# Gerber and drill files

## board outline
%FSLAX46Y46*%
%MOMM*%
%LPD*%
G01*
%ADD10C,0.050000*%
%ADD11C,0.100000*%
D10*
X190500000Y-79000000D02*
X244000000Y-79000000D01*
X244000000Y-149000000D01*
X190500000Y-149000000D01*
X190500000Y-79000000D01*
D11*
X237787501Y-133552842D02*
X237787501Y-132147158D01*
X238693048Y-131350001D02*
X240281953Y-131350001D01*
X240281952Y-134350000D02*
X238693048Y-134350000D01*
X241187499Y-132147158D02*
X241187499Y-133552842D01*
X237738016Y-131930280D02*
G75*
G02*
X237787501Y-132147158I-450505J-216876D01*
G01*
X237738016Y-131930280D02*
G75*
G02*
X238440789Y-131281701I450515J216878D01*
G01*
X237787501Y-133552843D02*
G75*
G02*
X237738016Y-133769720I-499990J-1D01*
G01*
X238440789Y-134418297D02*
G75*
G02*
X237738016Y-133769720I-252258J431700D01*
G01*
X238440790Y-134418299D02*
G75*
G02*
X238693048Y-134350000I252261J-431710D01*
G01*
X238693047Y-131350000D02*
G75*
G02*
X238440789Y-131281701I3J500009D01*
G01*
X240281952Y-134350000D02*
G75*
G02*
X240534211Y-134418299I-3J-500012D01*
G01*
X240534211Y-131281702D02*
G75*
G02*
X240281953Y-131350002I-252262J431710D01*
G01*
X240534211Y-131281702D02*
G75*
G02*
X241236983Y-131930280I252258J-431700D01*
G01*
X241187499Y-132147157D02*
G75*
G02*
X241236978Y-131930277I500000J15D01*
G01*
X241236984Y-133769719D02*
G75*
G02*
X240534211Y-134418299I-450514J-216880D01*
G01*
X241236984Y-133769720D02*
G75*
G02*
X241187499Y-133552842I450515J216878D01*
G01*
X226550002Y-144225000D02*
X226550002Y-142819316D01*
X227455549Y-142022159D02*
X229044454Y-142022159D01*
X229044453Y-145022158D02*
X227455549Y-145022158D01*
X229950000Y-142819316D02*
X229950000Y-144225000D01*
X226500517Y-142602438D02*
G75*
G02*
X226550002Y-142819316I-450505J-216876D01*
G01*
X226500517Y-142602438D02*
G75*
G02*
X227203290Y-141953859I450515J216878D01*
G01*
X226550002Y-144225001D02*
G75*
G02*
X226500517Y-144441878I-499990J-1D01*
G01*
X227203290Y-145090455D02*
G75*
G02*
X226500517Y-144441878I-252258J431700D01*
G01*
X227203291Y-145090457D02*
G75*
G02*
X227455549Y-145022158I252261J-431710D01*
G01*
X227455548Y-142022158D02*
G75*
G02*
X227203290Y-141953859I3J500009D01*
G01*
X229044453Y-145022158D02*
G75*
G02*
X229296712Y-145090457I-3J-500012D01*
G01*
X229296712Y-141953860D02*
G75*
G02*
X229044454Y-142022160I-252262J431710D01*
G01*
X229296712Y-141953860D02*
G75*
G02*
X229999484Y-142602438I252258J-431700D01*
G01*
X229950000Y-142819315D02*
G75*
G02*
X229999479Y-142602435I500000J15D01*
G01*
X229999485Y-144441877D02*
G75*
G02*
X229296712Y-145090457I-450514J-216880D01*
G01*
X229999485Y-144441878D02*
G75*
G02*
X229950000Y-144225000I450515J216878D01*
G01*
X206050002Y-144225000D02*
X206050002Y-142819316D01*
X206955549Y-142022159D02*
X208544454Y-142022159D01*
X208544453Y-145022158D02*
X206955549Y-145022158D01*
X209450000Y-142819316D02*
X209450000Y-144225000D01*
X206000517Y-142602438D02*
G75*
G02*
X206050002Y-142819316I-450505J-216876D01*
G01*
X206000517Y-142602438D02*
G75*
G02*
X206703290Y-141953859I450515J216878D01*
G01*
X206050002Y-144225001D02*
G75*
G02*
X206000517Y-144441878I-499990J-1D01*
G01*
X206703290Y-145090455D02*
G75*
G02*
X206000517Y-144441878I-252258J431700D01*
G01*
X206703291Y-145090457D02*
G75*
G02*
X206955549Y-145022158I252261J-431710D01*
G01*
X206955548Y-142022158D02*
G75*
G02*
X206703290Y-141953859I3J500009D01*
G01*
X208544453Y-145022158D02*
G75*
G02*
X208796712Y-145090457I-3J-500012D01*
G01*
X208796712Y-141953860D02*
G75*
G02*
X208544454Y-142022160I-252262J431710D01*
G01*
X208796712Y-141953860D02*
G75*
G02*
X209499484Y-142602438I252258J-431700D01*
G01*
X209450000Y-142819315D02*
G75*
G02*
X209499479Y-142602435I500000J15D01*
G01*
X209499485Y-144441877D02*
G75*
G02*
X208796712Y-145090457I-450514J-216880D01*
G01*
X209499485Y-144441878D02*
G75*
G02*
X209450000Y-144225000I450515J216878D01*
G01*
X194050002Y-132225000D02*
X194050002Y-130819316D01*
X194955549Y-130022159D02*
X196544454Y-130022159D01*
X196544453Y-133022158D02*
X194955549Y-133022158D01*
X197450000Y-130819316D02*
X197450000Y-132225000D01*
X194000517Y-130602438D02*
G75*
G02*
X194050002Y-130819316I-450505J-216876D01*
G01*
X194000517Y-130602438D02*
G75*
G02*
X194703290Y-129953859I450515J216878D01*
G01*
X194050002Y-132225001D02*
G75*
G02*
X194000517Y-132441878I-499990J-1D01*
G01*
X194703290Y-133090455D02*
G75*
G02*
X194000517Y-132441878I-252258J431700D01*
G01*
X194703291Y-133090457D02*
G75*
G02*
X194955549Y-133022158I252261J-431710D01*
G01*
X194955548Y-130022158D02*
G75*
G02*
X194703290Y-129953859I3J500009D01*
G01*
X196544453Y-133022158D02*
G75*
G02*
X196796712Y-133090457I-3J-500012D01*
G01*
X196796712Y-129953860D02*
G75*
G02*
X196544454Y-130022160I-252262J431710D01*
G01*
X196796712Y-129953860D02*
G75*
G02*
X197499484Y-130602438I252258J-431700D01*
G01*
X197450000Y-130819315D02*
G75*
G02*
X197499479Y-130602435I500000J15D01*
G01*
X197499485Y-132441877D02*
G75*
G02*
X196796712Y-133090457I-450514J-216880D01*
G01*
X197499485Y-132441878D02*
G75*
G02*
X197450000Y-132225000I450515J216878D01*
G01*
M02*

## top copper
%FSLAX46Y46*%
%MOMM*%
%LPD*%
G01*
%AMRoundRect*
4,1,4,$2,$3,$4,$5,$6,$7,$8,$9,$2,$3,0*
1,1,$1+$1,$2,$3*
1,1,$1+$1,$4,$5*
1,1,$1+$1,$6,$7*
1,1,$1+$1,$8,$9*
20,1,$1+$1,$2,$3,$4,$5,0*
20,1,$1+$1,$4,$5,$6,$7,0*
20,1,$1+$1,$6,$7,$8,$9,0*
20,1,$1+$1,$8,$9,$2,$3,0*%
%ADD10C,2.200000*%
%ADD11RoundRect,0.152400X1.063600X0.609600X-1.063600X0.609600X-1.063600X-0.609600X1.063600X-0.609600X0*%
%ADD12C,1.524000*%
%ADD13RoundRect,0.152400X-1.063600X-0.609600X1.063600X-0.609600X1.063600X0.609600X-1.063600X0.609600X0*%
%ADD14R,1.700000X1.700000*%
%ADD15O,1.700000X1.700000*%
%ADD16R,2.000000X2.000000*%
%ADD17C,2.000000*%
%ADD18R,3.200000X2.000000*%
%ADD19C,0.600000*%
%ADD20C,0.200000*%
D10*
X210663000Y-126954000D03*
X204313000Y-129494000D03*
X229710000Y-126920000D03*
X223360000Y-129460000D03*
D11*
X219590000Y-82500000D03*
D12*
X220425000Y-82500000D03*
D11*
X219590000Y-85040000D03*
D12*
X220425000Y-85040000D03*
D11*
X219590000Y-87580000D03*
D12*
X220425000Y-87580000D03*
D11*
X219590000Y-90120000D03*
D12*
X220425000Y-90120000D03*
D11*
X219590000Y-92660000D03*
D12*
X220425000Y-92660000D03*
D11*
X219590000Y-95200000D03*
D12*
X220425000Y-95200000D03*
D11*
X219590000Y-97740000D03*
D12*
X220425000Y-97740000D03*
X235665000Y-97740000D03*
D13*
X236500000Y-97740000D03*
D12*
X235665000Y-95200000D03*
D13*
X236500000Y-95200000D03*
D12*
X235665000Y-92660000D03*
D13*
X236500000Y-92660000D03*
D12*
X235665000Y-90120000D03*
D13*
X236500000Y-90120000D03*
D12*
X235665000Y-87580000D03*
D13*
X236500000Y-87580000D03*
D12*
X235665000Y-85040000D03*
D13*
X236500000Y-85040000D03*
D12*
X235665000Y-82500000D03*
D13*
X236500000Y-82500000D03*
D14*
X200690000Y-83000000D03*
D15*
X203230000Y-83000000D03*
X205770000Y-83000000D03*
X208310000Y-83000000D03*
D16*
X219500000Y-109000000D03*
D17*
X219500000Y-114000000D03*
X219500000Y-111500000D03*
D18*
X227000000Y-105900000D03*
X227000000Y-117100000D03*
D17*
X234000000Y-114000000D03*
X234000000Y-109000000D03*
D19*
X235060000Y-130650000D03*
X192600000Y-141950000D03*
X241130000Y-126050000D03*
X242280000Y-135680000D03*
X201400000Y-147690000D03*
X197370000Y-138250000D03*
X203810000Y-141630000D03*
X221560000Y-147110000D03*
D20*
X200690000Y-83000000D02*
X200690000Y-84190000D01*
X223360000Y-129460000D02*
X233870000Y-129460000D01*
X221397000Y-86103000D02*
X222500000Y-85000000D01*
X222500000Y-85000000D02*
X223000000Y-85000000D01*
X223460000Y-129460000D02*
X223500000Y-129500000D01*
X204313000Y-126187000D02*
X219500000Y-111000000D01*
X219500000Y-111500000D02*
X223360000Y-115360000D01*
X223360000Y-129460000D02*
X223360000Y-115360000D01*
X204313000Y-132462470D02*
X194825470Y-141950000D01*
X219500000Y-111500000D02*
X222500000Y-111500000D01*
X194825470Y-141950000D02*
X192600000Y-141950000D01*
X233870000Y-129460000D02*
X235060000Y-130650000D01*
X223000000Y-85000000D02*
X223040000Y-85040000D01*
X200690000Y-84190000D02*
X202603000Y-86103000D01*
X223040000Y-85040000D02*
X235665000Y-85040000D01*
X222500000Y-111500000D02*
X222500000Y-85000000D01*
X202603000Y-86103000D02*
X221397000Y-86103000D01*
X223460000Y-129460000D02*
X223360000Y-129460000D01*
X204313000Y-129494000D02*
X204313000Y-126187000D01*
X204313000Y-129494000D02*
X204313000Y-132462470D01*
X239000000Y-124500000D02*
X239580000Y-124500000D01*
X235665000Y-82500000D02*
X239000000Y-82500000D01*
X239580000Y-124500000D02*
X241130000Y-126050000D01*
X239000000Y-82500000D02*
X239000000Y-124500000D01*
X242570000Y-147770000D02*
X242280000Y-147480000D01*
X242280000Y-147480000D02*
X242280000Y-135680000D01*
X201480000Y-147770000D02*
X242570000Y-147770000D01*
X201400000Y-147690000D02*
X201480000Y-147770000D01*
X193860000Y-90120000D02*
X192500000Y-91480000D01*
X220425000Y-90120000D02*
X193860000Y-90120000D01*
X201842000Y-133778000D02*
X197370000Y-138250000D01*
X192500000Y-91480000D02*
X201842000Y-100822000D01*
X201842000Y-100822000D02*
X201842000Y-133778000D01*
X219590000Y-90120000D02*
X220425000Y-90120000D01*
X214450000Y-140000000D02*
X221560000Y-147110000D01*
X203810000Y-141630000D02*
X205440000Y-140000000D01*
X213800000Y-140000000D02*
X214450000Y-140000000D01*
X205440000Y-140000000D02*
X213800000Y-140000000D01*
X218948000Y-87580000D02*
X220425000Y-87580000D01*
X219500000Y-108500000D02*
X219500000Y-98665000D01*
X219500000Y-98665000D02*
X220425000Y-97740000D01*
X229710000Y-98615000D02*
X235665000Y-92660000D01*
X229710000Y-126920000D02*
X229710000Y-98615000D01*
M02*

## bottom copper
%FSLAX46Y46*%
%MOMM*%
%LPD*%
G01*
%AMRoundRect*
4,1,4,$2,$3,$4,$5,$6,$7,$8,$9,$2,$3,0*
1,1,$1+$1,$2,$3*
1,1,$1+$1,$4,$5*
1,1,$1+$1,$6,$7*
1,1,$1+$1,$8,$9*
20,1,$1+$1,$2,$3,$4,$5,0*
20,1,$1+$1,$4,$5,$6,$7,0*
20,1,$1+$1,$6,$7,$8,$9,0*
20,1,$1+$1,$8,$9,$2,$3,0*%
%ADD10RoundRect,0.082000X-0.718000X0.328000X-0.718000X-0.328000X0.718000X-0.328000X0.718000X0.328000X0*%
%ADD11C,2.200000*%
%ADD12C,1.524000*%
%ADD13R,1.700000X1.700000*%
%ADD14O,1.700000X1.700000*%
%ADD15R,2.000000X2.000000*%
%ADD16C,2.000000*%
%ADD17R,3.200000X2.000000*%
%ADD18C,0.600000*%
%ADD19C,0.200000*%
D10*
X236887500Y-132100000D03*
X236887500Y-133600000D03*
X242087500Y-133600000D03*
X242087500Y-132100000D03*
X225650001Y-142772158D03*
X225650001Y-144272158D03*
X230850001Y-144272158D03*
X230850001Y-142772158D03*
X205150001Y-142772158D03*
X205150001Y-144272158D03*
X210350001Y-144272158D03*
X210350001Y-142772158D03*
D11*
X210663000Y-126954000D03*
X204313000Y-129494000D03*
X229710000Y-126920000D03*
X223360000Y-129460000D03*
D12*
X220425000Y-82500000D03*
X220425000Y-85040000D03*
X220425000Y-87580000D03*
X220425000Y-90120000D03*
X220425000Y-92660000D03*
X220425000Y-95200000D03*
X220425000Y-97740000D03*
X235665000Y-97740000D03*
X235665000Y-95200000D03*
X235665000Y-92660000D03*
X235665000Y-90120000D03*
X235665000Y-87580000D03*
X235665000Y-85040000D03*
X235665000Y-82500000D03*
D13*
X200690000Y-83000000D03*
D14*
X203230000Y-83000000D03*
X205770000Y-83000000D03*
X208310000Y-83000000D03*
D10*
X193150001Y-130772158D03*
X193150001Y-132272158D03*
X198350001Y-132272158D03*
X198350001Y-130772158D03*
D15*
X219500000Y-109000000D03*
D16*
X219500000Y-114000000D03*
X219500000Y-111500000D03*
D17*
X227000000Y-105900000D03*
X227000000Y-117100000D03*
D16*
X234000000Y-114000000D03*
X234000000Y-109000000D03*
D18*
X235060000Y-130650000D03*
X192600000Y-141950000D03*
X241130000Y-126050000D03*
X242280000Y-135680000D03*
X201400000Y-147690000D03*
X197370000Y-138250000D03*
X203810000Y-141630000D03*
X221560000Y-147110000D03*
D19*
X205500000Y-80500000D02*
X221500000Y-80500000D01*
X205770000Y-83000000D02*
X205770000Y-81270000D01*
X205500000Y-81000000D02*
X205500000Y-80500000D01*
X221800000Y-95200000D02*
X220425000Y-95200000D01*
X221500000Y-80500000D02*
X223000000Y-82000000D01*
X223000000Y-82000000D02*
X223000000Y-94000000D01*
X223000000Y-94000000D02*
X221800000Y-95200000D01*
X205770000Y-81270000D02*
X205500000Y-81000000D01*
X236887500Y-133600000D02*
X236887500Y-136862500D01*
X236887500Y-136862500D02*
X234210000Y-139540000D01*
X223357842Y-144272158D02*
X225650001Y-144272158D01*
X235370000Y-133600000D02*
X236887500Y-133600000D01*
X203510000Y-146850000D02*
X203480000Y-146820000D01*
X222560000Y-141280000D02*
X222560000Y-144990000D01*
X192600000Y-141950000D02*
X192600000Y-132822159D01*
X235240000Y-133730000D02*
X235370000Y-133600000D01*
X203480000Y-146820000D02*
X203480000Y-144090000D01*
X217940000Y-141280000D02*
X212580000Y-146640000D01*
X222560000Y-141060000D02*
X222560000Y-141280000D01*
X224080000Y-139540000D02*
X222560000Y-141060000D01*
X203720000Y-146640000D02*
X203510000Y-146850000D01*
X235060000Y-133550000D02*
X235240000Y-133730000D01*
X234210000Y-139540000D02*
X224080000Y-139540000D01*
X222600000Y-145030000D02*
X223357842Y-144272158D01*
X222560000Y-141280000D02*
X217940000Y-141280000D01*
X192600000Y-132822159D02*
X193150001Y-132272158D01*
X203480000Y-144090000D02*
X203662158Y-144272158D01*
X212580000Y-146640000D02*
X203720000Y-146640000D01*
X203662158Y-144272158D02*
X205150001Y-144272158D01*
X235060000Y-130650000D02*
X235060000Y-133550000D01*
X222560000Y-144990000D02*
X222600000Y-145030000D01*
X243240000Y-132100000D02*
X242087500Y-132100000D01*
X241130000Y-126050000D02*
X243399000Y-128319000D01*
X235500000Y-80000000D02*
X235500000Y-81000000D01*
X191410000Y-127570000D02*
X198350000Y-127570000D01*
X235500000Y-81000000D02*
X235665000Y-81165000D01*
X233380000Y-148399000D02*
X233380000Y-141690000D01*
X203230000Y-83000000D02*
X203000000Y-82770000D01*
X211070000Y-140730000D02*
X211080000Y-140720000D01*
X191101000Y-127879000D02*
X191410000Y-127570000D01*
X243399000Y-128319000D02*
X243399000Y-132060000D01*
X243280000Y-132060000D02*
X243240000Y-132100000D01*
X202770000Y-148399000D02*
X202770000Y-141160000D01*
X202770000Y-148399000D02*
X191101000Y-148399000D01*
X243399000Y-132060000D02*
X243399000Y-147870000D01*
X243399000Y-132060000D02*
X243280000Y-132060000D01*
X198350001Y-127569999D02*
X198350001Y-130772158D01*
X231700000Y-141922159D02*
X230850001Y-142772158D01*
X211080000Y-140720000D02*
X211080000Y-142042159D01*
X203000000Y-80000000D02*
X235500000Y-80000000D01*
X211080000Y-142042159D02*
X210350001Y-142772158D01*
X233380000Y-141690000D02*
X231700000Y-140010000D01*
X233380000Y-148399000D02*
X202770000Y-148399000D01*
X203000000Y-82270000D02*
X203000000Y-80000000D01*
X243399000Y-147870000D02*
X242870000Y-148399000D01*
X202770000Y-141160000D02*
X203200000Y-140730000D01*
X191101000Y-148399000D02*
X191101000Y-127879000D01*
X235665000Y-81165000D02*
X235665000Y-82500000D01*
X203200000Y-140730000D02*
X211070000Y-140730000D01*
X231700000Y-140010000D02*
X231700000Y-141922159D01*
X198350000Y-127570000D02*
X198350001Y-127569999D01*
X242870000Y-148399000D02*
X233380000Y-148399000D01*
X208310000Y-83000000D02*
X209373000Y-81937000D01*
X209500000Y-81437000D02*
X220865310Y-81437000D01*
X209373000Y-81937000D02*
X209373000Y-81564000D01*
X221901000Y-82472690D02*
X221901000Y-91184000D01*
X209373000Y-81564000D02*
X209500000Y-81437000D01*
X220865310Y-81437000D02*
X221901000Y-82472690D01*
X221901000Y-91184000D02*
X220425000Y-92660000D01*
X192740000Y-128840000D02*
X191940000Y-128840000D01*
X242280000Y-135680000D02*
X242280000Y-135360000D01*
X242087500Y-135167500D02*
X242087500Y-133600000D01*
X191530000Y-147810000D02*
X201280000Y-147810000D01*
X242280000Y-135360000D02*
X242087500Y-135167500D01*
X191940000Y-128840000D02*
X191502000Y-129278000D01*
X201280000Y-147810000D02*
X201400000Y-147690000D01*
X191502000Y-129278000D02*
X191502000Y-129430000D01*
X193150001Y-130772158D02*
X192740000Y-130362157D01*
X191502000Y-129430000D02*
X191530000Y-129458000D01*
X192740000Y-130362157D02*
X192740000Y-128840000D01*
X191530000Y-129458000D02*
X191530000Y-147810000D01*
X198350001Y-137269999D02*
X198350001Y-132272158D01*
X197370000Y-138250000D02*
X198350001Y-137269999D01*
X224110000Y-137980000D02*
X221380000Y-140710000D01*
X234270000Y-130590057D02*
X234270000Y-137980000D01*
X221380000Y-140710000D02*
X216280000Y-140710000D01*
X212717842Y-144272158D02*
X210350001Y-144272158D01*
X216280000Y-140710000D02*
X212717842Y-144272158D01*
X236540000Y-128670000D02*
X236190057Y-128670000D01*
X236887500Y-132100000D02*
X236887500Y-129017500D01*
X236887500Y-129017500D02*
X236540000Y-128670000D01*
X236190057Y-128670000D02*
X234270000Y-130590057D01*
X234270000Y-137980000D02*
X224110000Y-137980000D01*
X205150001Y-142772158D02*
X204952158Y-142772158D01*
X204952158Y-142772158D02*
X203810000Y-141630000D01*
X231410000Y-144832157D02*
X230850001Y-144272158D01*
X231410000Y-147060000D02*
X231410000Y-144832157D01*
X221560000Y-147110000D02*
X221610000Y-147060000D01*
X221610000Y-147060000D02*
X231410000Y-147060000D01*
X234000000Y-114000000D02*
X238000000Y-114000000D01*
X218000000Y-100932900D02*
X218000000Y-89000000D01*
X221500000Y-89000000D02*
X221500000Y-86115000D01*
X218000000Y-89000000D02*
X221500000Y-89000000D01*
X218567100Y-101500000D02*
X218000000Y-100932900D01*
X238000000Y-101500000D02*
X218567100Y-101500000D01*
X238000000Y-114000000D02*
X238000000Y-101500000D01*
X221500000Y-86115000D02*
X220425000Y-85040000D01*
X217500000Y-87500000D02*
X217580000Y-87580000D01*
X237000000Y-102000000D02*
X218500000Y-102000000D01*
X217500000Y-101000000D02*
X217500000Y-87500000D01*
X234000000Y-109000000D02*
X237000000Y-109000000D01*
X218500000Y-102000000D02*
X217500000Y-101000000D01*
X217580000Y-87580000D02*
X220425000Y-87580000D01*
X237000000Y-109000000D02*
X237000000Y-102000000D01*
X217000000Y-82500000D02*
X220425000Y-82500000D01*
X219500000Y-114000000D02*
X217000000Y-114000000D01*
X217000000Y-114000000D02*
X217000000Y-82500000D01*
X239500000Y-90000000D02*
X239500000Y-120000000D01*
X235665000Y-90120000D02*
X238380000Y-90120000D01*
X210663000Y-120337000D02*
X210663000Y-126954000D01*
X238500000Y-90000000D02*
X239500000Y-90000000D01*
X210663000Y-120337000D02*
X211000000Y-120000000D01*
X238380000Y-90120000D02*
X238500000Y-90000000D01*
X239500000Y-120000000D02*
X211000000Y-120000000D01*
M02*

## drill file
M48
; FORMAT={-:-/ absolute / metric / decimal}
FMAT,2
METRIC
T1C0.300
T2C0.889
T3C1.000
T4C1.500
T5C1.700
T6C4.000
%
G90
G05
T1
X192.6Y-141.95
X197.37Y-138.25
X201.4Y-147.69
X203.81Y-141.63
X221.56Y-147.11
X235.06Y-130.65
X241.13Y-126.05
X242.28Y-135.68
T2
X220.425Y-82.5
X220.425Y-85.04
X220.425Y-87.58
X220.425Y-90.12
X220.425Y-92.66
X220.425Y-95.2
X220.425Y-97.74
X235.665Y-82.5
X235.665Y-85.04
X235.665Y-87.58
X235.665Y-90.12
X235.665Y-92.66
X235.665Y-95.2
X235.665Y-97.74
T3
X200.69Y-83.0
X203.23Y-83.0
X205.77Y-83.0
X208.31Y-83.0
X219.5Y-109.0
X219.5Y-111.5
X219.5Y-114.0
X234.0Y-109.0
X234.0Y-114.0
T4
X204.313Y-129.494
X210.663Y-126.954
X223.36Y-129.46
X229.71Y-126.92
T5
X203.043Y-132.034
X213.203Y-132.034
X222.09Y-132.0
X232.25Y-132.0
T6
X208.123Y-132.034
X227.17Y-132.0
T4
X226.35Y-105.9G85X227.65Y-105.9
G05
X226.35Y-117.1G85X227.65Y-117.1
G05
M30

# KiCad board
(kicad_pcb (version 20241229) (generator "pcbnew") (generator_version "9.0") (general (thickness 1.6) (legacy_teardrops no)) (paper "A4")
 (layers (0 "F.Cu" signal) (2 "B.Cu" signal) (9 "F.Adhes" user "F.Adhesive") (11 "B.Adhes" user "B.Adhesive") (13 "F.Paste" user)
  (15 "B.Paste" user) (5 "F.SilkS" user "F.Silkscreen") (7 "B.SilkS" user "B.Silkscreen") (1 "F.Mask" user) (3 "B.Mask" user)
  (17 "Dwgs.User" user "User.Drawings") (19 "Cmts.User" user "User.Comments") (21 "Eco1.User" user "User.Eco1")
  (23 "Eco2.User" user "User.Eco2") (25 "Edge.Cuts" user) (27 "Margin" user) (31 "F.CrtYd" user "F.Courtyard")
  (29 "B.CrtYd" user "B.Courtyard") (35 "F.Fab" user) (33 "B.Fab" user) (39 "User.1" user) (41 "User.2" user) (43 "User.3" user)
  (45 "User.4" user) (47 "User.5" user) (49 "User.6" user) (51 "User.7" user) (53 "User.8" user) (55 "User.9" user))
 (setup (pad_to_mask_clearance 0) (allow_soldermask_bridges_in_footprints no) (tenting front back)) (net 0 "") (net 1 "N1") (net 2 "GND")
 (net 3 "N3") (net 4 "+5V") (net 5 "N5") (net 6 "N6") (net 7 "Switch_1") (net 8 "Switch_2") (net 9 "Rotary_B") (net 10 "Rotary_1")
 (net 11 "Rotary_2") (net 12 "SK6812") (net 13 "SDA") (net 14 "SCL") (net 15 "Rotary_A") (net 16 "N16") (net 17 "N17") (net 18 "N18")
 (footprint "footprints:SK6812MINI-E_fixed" (layer "F.Cu") (at 239.487499 132.952842)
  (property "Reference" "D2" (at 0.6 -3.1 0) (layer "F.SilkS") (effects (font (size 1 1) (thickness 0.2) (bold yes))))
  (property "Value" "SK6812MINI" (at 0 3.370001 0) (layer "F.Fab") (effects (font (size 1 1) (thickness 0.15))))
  (fp_line (start -1.699998 0.6) (end -1.699998 -0.805684) (stroke (width 0.1) (type solid)) (layer "Edge.Cuts"))
  (fp_line (start -0.794451 -1.602841) (end 0.794454 -1.602841) (stroke (width 0.1) (type solid)) (layer "Edge.Cuts"))
  (fp_line (start 0.794453 1.397158) (end -0.794451 1.397158) (stroke (width 0.1) (type solid)) (layer "Edge.Cuts"))
  (fp_line (start 1.7 -0.805684) (end 1.7 0.6) (stroke (width 0.1) (type solid)) (layer "Edge.Cuts"))
  (fp_arc (start -1.749483 -1.022562) (mid -1.712526 -0.91691) (end -1.699998 -0.805684) (stroke (width 0.1) (type solid))
   (layer "Edge.Cuts"))
  (fp_arc (start -1.749483 -1.022562) (mid -1.63807 -1.606877) (end -1.04671 -1.671141) (stroke (width 0.1) (type solid))
   (layer "Edge.Cuts"))
  (fp_arc (start -1.699998 0.600001) (mid -1.712526 0.711226) (end -1.749483 0.816878) (stroke (width 0.1) (type solid)) (layer "Edge.Cuts"))
  (fp_arc (start -1.04671 1.465455) (mid -1.638069 1.401192) (end -1.749483 0.816878) (stroke (width 0.1) (type solid)) (layer "Edge.Cuts"))
  (fp_arc (start -1.046709 1.465457) (mid -0.925121 1.414535) (end -0.794451 1.397158) (stroke (width 0.1) (type solid)) (layer "Edge.Cuts"))
  (fp_arc (start -0.794452 -1.602842) (mid -0.925122 -1.620219) (end -1.04671 -1.671141) (stroke (width 0.1) (type solid))
   (layer "Edge.Cuts"))
  (fp_arc (start 0.794453 1.397158) (mid 0.925124 1.414535) (end 1.046712 1.465457) (stroke (width 0.1) (type solid)) (layer "Edge.Cuts"))
  (fp_arc (start 1.046712 -1.67114) (mid 0.925124 -1.620218) (end 0.794454 -1.602841) (stroke (width 0.1) (type solid)) (layer "Edge.Cuts"))
  (fp_arc (start 1.046712 -1.67114) (mid 1.638072 -1.606876) (end 1.749485 -1.022562) (stroke (width 0.1) (type solid)) (layer "Edge.Cuts"))
  (fp_arc (start 1.7 -0.805685) (mid 1.712528 -0.91691) (end 1.749485 -1.022562) (stroke (width 0.1) (type solid)) (layer "Edge.Cuts"))
  (fp_arc (start 1.749485 0.816877) (mid 1.638073 1.401193) (end 1.046712 1.465457) (stroke (width 0.1) (type solid)) (layer "Edge.Cuts"))
  (fp_arc (start 1.749485 0.816878) (mid 1.712528 0.711226) (end 1.7 0.6) (stroke (width 0.1) (type solid)) (layer "Edge.Cuts"))
  (pad "1" smd roundrect (at -2.599999 -0.852842 270) (size 0.82 1.6) (layers "B.Cu" "B.Mask" "B.Paste") (roundrect_rratio 0.1) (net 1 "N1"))
  (pad "2" smd roundrect (at -2.599999 0.647158 270) (size 0.82 1.6) (layers "B.Cu" "B.Mask" "B.Paste") (roundrect_rratio 0.1) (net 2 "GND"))
  (pad "3" smd roundrect (at 2.600001 0.647158 270) (size 0.82 1.6) (layers "B.Cu" "B.Mask" "B.Paste") (roundrect_rratio 0.1) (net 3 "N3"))
  (pad "4" smd roundrect (at 2.600001 -0.852842 270) (size 0.82 1.6) (layers "B.Cu" "B.Mask" "B.Paste") (roundrect_rratio 0.1) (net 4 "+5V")))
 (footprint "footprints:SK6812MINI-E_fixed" (layer "F.Cu") (at 228.25 143.625)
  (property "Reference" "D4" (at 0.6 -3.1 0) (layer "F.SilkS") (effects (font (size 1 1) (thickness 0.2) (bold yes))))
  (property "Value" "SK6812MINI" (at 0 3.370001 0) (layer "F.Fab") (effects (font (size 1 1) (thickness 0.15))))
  (fp_line (start -1.699998 0.6) (end -1.699998 -0.805684) (stroke (width 0.1) (type solid)) (layer "Edge.Cuts"))
  (fp_line (start -0.794451 -1.602841) (end 0.794454 -1.602841) (stroke (width 0.1) (type solid)) (layer "Edge.Cuts"))
  (fp_line (start 0.794453 1.397158) (end -0.794451 1.397158) (stroke (width 0.1) (type solid)) (layer "Edge.Cuts"))
  (fp_line (start 1.7 -0.805684) (end 1.7 0.6) (stroke (width 0.1) (type solid)) (layer "Edge.Cuts"))
  (fp_arc (start -1.749483 -1.022562) (mid -1.712526 -0.91691) (end -1.699998 -0.805684) (stroke (width 0.1) (type solid))
   (layer "Edge.Cuts"))
  (fp_arc (start -1.749483 -1.022562) (mid -1.63807 -1.606877) (end -1.04671 -1.671141) (stroke (width 0.1) (type solid))
   (layer "Edge.Cuts"))
  (fp_arc (start -1.699998 0.600001) (mid -1.712526 0.711226) (end -1.749483 0.816878) (stroke (width 0.1) (type solid)) (layer "Edge.Cuts"))
  (fp_arc (start -1.04671 1.465455) (mid -1.638069 1.401192) (end -1.749483 0.816878) (stroke (width 0.1) (type solid)) (layer "Edge.Cuts"))
  (fp_arc (start -1.046709 1.465457) (mid -0.925121 1.414535) (end -0.794451 1.397158) (stroke (width 0.1) (type solid)) (layer "Edge.Cuts"))
  (fp_arc (start -0.794452 -1.602842) (mid -0.925122 -1.620219) (end -1.04671 -1.671141) (stroke (width 0.1) (type solid))
   (layer "Edge.Cuts"))
  (fp_arc (start 0.794453 1.397158) (mid 0.925124 1.414535) (end 1.046712 1.465457) (stroke (width 0.1) (type solid)) (layer "Edge.Cuts"))
  (fp_arc (start 1.046712 -1.67114) (mid 0.925124 -1.620218) (end 0.794454 -1.602841) (stroke (width 0.1) (type solid)) (layer "Edge.Cuts"))
  (fp_arc (start 1.046712 -1.67114) (mid 1.638072 -1.606876) (end 1.749485 -1.022562) (stroke (width 0.1) (type solid)) (layer "Edge.Cuts"))
  (fp_arc (start 1.7 -0.805685) (mid 1.712528 -0.91691) (end 1.749485 -1.022562) (stroke (width 0.1) (type solid)) (layer "Edge.Cuts"))
  (fp_arc (start 1.749485 0.816877) (mid 1.638073 1.401193) (end 1.046712 1.465457) (stroke (width 0.1) (type solid)) (layer "Edge.Cuts"))
  (fp_arc (start 1.749485 0.816878) (mid 1.712528 0.711226) (end 1.7 0.6) (stroke (width 0.1) (type solid)) (layer "Edge.Cuts"))
  (pad "1" smd roundrect (at -2.599999 -0.852842 270) (size 0.82 1.6) (layers "B.Cu" "B.Mask" "B.Paste") (roundrect_rratio 0.1) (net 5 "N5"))
  (pad "2" smd roundrect (at -2.599999 0.647158 270) (size 0.82 1.6) (layers "B.Cu" "B.Mask" "B.Paste") (roundrect_rratio 0.1) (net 2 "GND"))
  (pad "3" smd roundrect (at 2.600001 0.647158 270) (size 0.82 1.6) (layers "B.Cu" "B.Mask" "B.Paste") (roundrect_rratio 0.1) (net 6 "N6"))
  (pad "4" smd roundrect (at 2.600001 -0.852842 270) (size 0.82 1.6) (layers "B.Cu" "B.Mask" "B.Paste") (roundrect_rratio 0.1) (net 4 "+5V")))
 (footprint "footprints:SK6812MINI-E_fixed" (layer "F.Cu") (at 207.75 143.625)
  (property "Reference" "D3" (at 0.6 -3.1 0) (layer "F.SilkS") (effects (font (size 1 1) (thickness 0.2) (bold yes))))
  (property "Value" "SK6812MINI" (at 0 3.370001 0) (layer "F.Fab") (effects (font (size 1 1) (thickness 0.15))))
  (fp_line (start -1.699998 0.6) (end -1.699998 -0.805684) (stroke (width 0.1) (type solid)) (layer "Edge.Cuts"))
  (fp_line (start -0.794451 -1.602841) (end 0.794454 -1.602841) (stroke (width 0.1) (type solid)) (layer "Edge.Cuts"))
  (fp_line (start 0.794453 1.397158) (end -0.794451 1.397158) (stroke (width 0.1) (type solid)) (layer "Edge.Cuts"))
  (fp_line (start 1.7 -0.805684) (end 1.7 0.6) (stroke (width 0.1) (type solid)) (layer "Edge.Cuts"))
  (fp_arc (start -1.749483 -1.022562) (mid -1.712526 -0.91691) (end -1.699998 -0.805684) (stroke (width 0.1) (type solid))
   (layer "Edge.Cuts"))
  (fp_arc (start -1.749483 -1.022562) (mid -1.63807 -1.606877) (end -1.04671 -1.671141) (stroke (width 0.1) (type solid))
   (layer "Edge.Cuts"))
  (fp_arc (start -1.699998 0.600001) (mid -1.712526 0.711226) (end -1.749483 0.816878) (stroke (width 0.1) (type solid)) (layer "Edge.Cuts"))
  (fp_arc (start -1.04671 1.465455) (mid -1.638069 1.401192) (end -1.749483 0.816878) (stroke (width 0.1) (type solid)) (layer "Edge.Cuts"))
  (fp_arc (start -1.046709 1.465457) (mid -0.925121 1.414535) (end -0.794451 1.397158) (stroke (width 0.1) (type solid)) (layer "Edge.Cuts"))
  (fp_arc (start -0.794452 -1.602842) (mid -0.925122 -1.620219) (end -1.04671 -1.671141) (stroke (width 0.1) (type solid))
   (layer "Edge.Cuts"))
  (fp_arc (start 0.794453 1.397158) (mid 0.925124 1.414535) (end 1.046712 1.465457) (stroke (width 0.1) (type solid)) (layer "Edge.Cuts"))
  (fp_arc (start 1.046712 -1.67114) (mid 0.925124 -1.620218) (end 0.794454 -1.602841) (stroke (width 0.1) (type solid)) (layer "Edge.Cuts"))
  (fp_arc (start 1.046712 -1.67114) (mid 1.638072 -1.606876) (end 1.749485 -1.022562) (stroke (width 0.1) (type solid)) (layer "Edge.Cuts"))
  (fp_arc (start 1.7 -0.805685) (mid 1.712528 -0.91691) (end 1.749485 -1.022562) (stroke (width 0.1) (type solid)) (layer "Edge.Cuts"))
  (fp_arc (start 1.749485 0.816877) (mid 1.638073 1.401193) (end 1.046712 1.465457) (stroke (width 0.1) (type solid)) (layer "Edge.Cuts"))
  (fp_arc (start 1.749485 0.816878) (mid 1.712528 0.711226) (end 1.7 0.6) (stroke (width 0.1) (type solid)) (layer "Edge.Cuts"))
  (pad "1" smd roundrect (at -2.599999 -0.852842 270) (size 0.82 1.6) (layers "B.Cu" "B.Mask" "B.Paste") (roundrect_rratio 0.1) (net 6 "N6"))
  (pad "2" smd roundrect (at -2.599999 0.647158 270) (size 0.82 1.6) (layers "B.Cu" "B.Mask" "B.Paste") (roundrect_rratio 0.1) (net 2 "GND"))
  (pad "3" smd roundrect (at 2.600001 0.647158 270) (size 0.82 1.6) (layers "B.Cu" "B.Mask" "B.Paste") (roundrect_rratio 0.1) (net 1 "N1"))
  (pad "4" smd roundrect (at 2.600001 -0.852842 270) (size 0.82 1.6) (layers "B.Cu" "B.Mask" "B.Paste") (roundrect_rratio 0.1) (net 4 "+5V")))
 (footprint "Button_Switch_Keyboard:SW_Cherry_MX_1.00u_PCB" (layer "F.Cu") (at 210.663 126.954)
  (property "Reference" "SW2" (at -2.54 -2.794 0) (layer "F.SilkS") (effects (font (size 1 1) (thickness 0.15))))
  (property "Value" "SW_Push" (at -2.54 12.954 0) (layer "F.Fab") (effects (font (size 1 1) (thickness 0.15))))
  (pad "" np_thru_hole circle (at -7.62 5.08) (size 1.7 1.7) (drill 1.7) (layers "*.Cu" "*.Mask"))
  (pad "" np_thru_hole circle (at -2.54 5.08) (size 4 4) (drill 4) (layers "*.Cu" "*.Mask"))
  (pad "" np_thru_hole circle (at 2.54 5.08) (size 1.7 1.7) (drill 1.7) (layers "*.Cu" "*.Mask"))
  (pad "1" thru_hole circle (at 0 0) (size 2.2 2.2) (drill 1.5) (layers "*.Cu" "*.Mask") (remove_unused_layers no) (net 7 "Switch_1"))
  (pad "2" thru_hole circle (at -6.35 2.54) (size 2.2 2.2) (drill 1.5) (layers "*.Cu" "*.Mask") (remove_unused_layers no) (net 2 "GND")))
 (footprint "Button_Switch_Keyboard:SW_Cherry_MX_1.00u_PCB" (layer "F.Cu") (at 229.71 126.92)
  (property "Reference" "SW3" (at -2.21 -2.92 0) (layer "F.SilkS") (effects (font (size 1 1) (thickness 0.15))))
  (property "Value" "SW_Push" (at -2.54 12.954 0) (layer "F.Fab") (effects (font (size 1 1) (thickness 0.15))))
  (pad "" np_thru_hole circle (at -7.62 5.08) (size 1.7 1.7) (drill 1.7) (layers "*.Cu" "*.Mask"))
  (pad "" np_thru_hole circle (at -2.54 5.08) (size 4 4) (drill 4) (layers "*.Cu" "*.Mask"))
  (pad "" np_thru_hole circle (at 2.54 5.08) (size 1.7 1.7) (drill 1.7) (layers "*.Cu" "*.Mask"))
  (pad "1" thru_hole circle (at 0 0) (size 2.2 2.2) (drill 1.5) (layers "*.Cu" "*.Mask") (remove_unused_layers no) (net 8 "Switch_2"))
  (pad "2" thru_hole circle (at -6.35 2.54) (size 2.2 2.2) (drill 1.5) (layers "*.Cu" "*.Mask") (remove_unused_layers no) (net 2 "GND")))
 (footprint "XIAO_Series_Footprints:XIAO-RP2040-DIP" (layer "F.Cu") (at 228.045 90.12 90)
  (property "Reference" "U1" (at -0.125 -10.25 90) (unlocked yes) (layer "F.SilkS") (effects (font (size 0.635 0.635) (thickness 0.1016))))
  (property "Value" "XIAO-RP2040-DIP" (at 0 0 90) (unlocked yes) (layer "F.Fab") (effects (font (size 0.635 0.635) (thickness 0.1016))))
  (pad "1" smd roundrect (at 7.62 -8.455 180) (size 2.432 1.524) (layers "F.Cu" "F.Mask") (roundrect_rratio 0.1) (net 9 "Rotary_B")
   (thermal_bridge_angle 45))
  (pad "1" thru_hole circle (at 7.62 -7.62 180) (size 1.524 1.524) (drill 0.889) (layers "*.Cu" "*.Mask") (remove_unused_layers no)
   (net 9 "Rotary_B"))
  (pad "2" smd roundrect (at 5.08 -8.455 180) (size 2.432 1.524) (layers "F.Cu" "F.Mask") (roundrect_rratio 0.1) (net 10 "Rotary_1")
   (thermal_bridge_angle 45))
  (pad "2" thru_hole circle (at 5.08 -7.62 180) (size 1.524 1.524) (drill 0.889) (layers "*.Cu" "*.Mask") (remove_unused_layers no)
   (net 10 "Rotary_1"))
  (pad "3" smd roundrect (at 2.54 -8.455 180) (size 2.432 1.524) (layers "F.Cu" "F.Mask") (roundrect_rratio 0.1) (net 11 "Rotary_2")
   (thermal_bridge_angle 45))
  (pad "3" thru_hole circle (at 2.54 -7.62 180) (size 1.524 1.524) (drill 0.889) (layers "*.Cu" "*.Mask") (remove_unused_layers no)
   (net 11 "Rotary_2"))
  (pad "4" smd roundrect (at 0 -8.455 180) (size 2.432 1.524) (layers "F.Cu" "F.Mask") (roundrect_rratio 0.1) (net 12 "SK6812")
   (thermal_bridge_angle 45))
  (pad "4" thru_hole circle (at 0 -7.62 180) (size 1.524 1.524) (drill 0.889) (layers "*.Cu" "*.Mask") (remove_unused_layers no)
   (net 12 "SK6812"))
  (pad "5" smd roundrect (at -2.54 -8.455 180) (size 2.432 1.524) (layers "F.Cu" "F.Mask") (roundrect_rratio 0.1) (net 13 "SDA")
   (thermal_bridge_angle 45))
  (pad "5" thru_hole circle (at -2.54 -7.62 180) (size 1.524 1.524) (drill 0.889) (layers "*.Cu" "*.Mask") (remove_unused_layers no)
   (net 13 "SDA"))
  (pad "6" smd roundrect (at -5.08 -8.455 180) (size 2.432 1.524) (layers "F.Cu" "F.Mask") (roundrect_rratio 0.1) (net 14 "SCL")
   (thermal_bridge_angle 45))
  (pad "6" thru_hole circle (at -5.08 -7.62 180) (size 1.524 1.524) (drill 0.889) (layers "*.Cu" "*.Mask") (remove_unused_layers no)
   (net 14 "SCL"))
  (pad "7" smd roundrect (at -7.62 -8.455 180) (size 2.432 1.524) (layers "F.Cu" "F.Mask") (roundrect_rratio 0.1) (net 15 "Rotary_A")
   (thermal_bridge_angle 45))
  (pad "7" thru_hole circle (at -7.62 -7.62 180) (size 1.524 1.524) (drill 0.889) (layers "*.Cu" "*.Mask") (remove_unused_layers no)
   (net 15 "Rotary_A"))
  (pad "8" thru_hole circle (at -7.62 7.62) (size 1.524 1.524) (drill 0.889) (layers "*.Cu" "*.Mask") (remove_unused_layers no)
   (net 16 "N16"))
  (pad "8" smd roundrect (at -7.62 8.455) (size 2.432 1.524) (layers "F.Cu" "F.Mask") (roundrect_rratio 0.1) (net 16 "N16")
   (thermal_bridge_angle 45))
  (pad "9" thru_hole circle (at -5.08 7.62) (size 1.524 1.524) (drill 0.889) (layers "*.Cu" "*.Mask") (remove_unused_layers no)
   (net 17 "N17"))
  (pad "9" smd roundrect (at -5.08 8.455) (size 2.432 1.524) (layers "F.Cu" "F.Mask") (roundrect_rratio 0.1) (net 17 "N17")
   (thermal_bridge_angle 45))
  (pad "10" thru_hole circle (at -2.54 7.62) (size 1.524 1.524) (drill 0.889) (layers "*.Cu" "*.Mask") (remove_unused_layers no)
   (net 8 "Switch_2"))
  (pad "10" smd roundrect (at -2.54 8.455) (size 2.432 1.524) (layers "F.Cu" "F.Mask") (roundrect_rratio 0.1) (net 8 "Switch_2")
   (thermal_bridge_angle 45))
  (pad "11" thru_hole circle (at 0 7.62) (size 1.524 1.524) (drill 0.889) (layers "*.Cu" "*.Mask") (remove_unused_layers no)
   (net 7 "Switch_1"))
  (pad "11" smd roundrect (at 0 8.455) (size 2.432 1.524) (layers "F.Cu" "F.Mask") (roundrect_rratio 0.1) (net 7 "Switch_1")
   (thermal_bridge_angle 45))
  (pad "12" thru_hole circle (at 2.54 7.62) (size 1.524 1.524) (drill 0.889) (layers "*.Cu" "*.Mask") (remove_unused_layers no)
   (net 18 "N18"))
  (pad "12" smd roundrect (at 2.54 8.455) (size 2.432 1.524) (layers "F.Cu" "F.Mask") (roundrect_rratio 0.1) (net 18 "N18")
   (thermal_bridge_angle 45))
  (pad "13" thru_hole circle (at 5.08 7.62) (size 1.524 1.524) (drill 0.889) (layers "*.Cu" "*.Mask") (remove_unused_layers no)
   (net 2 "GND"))
  (pad "13" smd roundrect (at 5.08 8.455) (size 2.432 1.524) (layers "F.Cu" "F.Mask") (roundrect_rratio 0.1) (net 2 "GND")
   (thermal_bridge_angle 45))
  (pad "14" thru_hole circle (at 7.62 7.62) (size 1.524 1.524) (drill 0.889) (layers "*.Cu" "*.Mask") (remove_unused_layers no)
   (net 4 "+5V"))
  (pad "14" smd roundrect (at 7.62 8.455) (size 2.432 1.524) (layers "F.Cu" "F.Mask") (roundrect_rratio 0.1) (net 4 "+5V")
   (thermal_bridge_angle 45)))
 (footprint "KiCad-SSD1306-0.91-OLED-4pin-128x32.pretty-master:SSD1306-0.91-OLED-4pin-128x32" (layer "F.Cu") (at 198.5 119.5 90)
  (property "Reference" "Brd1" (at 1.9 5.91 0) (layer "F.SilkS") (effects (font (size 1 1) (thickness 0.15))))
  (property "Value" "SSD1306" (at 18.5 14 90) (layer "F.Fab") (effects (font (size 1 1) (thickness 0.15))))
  (pad "1" thru_hole rect (at 36.5 2.19 90) (size 1.7 1.7) (drill 1) (layers "*.Cu" "*.Mask") (remove_unused_layers no) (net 2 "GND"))
  (pad "2" thru_hole oval (at 36.5 4.73 90) (size 1.7 1.7) (drill 1) (layers "*.Cu" "*.Mask") (remove_unused_layers no) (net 4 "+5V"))
  (pad "3" thru_hole oval (at 36.5 7.27 90) (size 1.7 1.7) (drill 1) (layers "*.Cu" "*.Mask") (remove_unused_layers no) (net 14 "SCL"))
  (pad "4" thru_hole oval (at 36.5 9.81 90) (size 1.7 1.7) (drill 1) (layers "*.Cu" "*.Mask") (remove_unused_layers no) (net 13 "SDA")))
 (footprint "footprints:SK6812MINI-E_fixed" (layer "F.Cu") (at 195.75 131.625)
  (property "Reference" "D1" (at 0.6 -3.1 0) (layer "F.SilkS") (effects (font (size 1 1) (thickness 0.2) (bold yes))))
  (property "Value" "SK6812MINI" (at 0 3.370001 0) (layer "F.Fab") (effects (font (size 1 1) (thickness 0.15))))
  (fp_line (start -1.699998 0.6) (end -1.699998 -0.805684) (stroke (width 0.1) (type solid)) (layer "Edge.Cuts"))
  (fp_line (start -0.794451 -1.602841) (end 0.794454 -1.602841) (stroke (width 0.1) (type solid)) (layer "Edge.Cuts"))
  (fp_line (start 0.794453 1.397158) (end -0.794451 1.397158) (stroke (width 0.1) (type solid)) (layer "Edge.Cuts"))
  (fp_line (start 1.7 -0.805684) (end 1.7 0.6) (stroke (width 0.1) (type solid)) (layer "Edge.Cuts"))
  (fp_arc (start -1.749483 -1.022562) (mid -1.712526 -0.91691) (end -1.699998 -0.805684) (stroke (width 0.1) (type solid))
   (layer "Edge.Cuts"))
  (fp_arc (start -1.749483 -1.022562) (mid -1.63807 -1.606877) (end -1.04671 -1.671141) (stroke (width 0.1) (type solid))
   (layer "Edge.Cuts"))
  (fp_arc (start -1.699998 0.600001) (mid -1.712526 0.711226) (end -1.749483 0.816878) (stroke (width 0.1) (type solid)) (layer "Edge.Cuts"))
  (fp_arc (start -1.04671 1.465455) (mid -1.638069 1.401192) (end -1.749483 0.816878) (stroke (width 0.1) (type solid)) (layer "Edge.Cuts"))
  (fp_arc (start -1.046709 1.465457) (mid -0.925121 1.414535) (end -0.794451 1.397158) (stroke (width 0.1) (type solid)) (layer "Edge.Cuts"))
  (fp_arc (start -0.794452 -1.602842) (mid -0.925122 -1.620219) (end -1.04671 -1.671141) (stroke (width 0.1) (type solid))
   (layer "Edge.Cuts"))
  (fp_arc (start 0.794453 1.397158) (mid 0.925124 1.414535) (end 1.046712 1.465457) (stroke (width 0.1) (type solid)) (layer "Edge.Cuts"))
  (fp_arc (start 1.046712 -1.67114) (mid 0.925124 -1.620218) (end 0.794454 -1.602841) (stroke (width 0.1) (type solid)) (layer "Edge.Cuts"))
  (fp_arc (start 1.046712 -1.67114) (mid 1.638072 -1.606876) (end 1.749485 -1.022562) (stroke (width 0.1) (type solid)) (layer "Edge.Cuts"))
  (fp_arc (start 1.7 -0.805685) (mid 1.712528 -0.91691) (end 1.749485 -1.022562) (stroke (width 0.1) (type solid)) (layer "Edge.Cuts"))
  (fp_arc (start 1.749485 0.816877) (mid 1.638073 1.401193) (end 1.046712 1.465457) (stroke (width 0.1) (type solid)) (layer "Edge.Cuts"))
  (fp_arc (start 1.749485 0.816878) (mid 1.712528 0.711226) (end 1.7 0.6) (stroke (width 0.1) (type solid)) (layer "Edge.Cuts"))
  (pad "1" smd roundrect (at -2.599999 -0.852842 270) (size 0.82 1.6) (layers "B.Cu" "B.Mask" "B.Paste") (roundrect_rratio 0.1) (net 3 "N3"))
  (pad "2" smd roundrect (at -2.599999 0.647158 270) (size 0.82 1.6) (layers "B.Cu" "B.Mask" "B.Paste") (roundrect_rratio 0.1) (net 2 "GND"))
  (pad "3" smd roundrect (at 2.600001 0.647158 270) (size 0.82 1.6) (layers "B.Cu" "B.Mask" "B.Paste") (roundrect_rratio 0.1)
   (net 12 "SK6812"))
  (pad "4" smd roundrect (at 2.600001 -0.852842 270) (size 0.82 1.6) (layers "B.Cu" "B.Mask" "B.Paste") (roundrect_rratio 0.1) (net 4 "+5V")))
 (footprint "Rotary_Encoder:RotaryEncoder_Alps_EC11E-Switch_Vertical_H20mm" (layer "F.Cu") (at 219.5 109)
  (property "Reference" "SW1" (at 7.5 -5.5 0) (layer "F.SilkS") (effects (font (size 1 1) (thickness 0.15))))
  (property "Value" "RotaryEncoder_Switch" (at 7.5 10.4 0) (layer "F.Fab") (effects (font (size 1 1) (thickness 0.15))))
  (pad "A" thru_hole rect (at 0 0) (size 2 2) (drill 1) (layers "*.Cu" "*.Mask") (remove_unused_layers no) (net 15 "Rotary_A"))
  (pad "B" thru_hole circle (at 0 5) (size 2 2) (drill 1) (layers "*.Cu" "*.Mask") (remove_unused_layers no) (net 9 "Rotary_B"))
  (pad "C" thru_hole circle (at 0 2.5) (size 2 2) (drill 1) (layers "*.Cu" "*.Mask") (remove_unused_layers no) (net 2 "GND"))
  (pad "MP" thru_hole rect (at 7.5 -3.1) (size 3.2 2) (drill oval 2.8 1.5) (layers "*.Cu" "*.Mask") (remove_unused_layers no))
  (pad "MP" thru_hole rect (at 7.5 8.1) (size 3.2 2) (drill oval 2.8 1.5) (layers "*.Cu" "*.Mask") (remove_unused_layers no))
  (pad "S1" thru_hole circle (at 14.5 5) (size 2 2) (drill 1) (layers "*.Cu" "*.Mask") (remove_unused_layers no) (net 10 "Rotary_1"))
  (pad "S2" thru_hole circle (at 14.5 0) (size 2 2) (drill 1) (layers "*.Cu" "*.Mask") (remove_unused_layers no) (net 11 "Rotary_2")))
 (gr_rect (start 190.5 79) (end 244 149) (stroke (width 0.05) (type default)) (fill no) (layer "Edge.Cuts"))
 (segment (start 205.5 80.5) (end 221.5 80.5) (width 0.2) (layer "B.Cu") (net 14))
 (segment (start 205.77 83) (end 205.77 81.27) (width 0.2) (layer "B.Cu") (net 14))
 (segment (start 205.5 81) (end 205.5 80.5) (width 0.2) (layer "B.Cu") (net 14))
 (segment (start 221.8 95.2) (end 220.425 95.2) (width 0.2) (layer "B.Cu") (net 14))
 (segment (start 221.5 80.5) (end 223 82) (width 0.2) (layer "B.Cu") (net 14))
 (segment (start 223 82) (end 223 94) (width 0.2) (layer "B.Cu") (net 14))
 (segment (start 223 94) (end 221.8 95.2) (width 0.2) (layer "B.Cu") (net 14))
 (segment (start 205.77 81.27) (end 205.5 81) (width 0.2) (layer "B.Cu") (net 14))
 (segment (start 200.69 83) (end 200.69 84.19) (width 0.2) (layer "F.Cu") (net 2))
 (segment (start 223.36 129.46) (end 233.87 129.46) (width 0.2) (layer "F.Cu") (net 2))
 (segment (start 221.397 86.103) (end 222.5 85) (width 0.2) (layer "F.Cu") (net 2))
 (segment (start 222.5 85) (end 223 85) (width 0.2) (layer "F.Cu") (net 2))
 (segment (start 223.46 129.46) (end 223.5 129.5) (width 0.2) (layer "F.Cu") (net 2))
 (segment (start 204.313 126.187) (end 219.5 111) (width 0.2) (layer "F.Cu") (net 2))
 (segment (start 219.5 111.5) (end 223.36 115.36) (width 0.2) (layer "F.Cu") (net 2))
 (segment (start 223.36 129.46) (end 223.36 115.36) (width 0.2) (layer "F.Cu") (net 2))
 (segment (start 204.313 132.46247) (end 194.82547 141.95) (width 0.2) (layer "F.Cu") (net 2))
 (segment (start 219.5 111.5) (end 222.5 111.5) (width 0.2) (layer "F.Cu") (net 2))
 (segment (start 194.82547 141.95) (end 192.6 141.95) (width 0.2) (layer "F.Cu") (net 2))
 (segment (start 233.87 129.46) (end 235.06 130.65) (width 0.2) (layer "F.Cu") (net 2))
 (segment (start 223 85) (end 223.04 85.04) (width 0.2) (layer "F.Cu") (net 2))
 (segment (start 200.69 84.19) (end 202.603 86.103) (width 0.2) (layer "F.Cu") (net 2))
 (segment (start 223.04 85.04) (end 235.665 85.04) (width 0.2) (layer "F.Cu") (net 2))
 (segment (start 222.5 111.5) (end 222.5 85) (width 0.2) (layer "F.Cu") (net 2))
 (segment (start 202.603 86.103) (end 221.397 86.103) (width 0.2) (layer "F.Cu") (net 2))
 (segment (start 223.46 129.46) (end 223.36 129.46) (width 0.2) (layer "F.Cu") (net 2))
 (segment (start 204.313 129.494) (end 204.313 126.187) (width 0.2) (layer "F.Cu") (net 2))
 (segment (start 204.313 129.494) (end 204.313 132.46247) (width 0.2) (layer "F.Cu") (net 2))
 (via (at 235.06 130.65) (size 0.6) (drill 0.3) (layers "F.Cu" "B.Cu") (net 2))
 (via (at 192.6 141.95) (size 0.6) (drill 0.3) (layers "F.Cu" "B.Cu") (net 2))
 (segment (start 236.8875 133.6) (end 236.8875 136.8625) (width 0.2) (layer "B.Cu") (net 2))
 (segment (start 236.8875 136.8625) (end 234.21 139.54) (width 0.2) (layer "B.Cu") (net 2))
 (segment (start 223.357842 144.272158) (end 225.650001 144.272158) (width 0.2) (layer "B.Cu") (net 2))
 (segment (start 235.37 133.6) (end 236.8875 133.6) (width 0.2) (layer "B.Cu") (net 2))
 (segment (start 203.51 146.85) (end 203.48 146.82) (width 0.2) (layer "B.Cu") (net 2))
 (segment (start 222.56 141.28) (end 222.56 144.99) (width 0.2) (layer "B.Cu") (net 2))
 (segment (start 192.6 141.95) (end 192.6 132.822159) (width 0.2) (layer "B.Cu") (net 2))
 (segment (start 235.24 133.73) (end 235.37 133.6) (width 0.2) (layer "B.Cu") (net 2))
 (segment (start 203.48 146.82) (end 203.48 144.09) (width 0.2) (layer "B.Cu") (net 2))
 (segment (start 217.94 141.28) (end 212.58 146.64) (width 0.2) (layer "B.Cu") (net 2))
 (segment (start 222.56 141.06) (end 222.56 141.28) (width 0.2) (layer "B.Cu") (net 2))
 (segment (start 224.08 139.54) (end 222.56 141.06) (width 0.2) (layer "B.Cu") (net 2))
 (segment (start 203.72 146.64) (end 203.51 146.85) (width 0.2) (layer "B.Cu") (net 2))
 (segment (start 235.06 133.55) (end 235.24 133.73) (width 0.2) (layer "B.Cu") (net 2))
 (segment (start 234.21 139.54) (end 224.08 139.54) (width 0.2) (layer "B.Cu") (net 2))
 (segment (start 222.6 145.03) (end 223.357842 144.272158) (width 0.2) (layer "B.Cu") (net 2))
 (segment (start 222.56 141.28) (end 217.94 141.28) (width 0.2) (layer "B.Cu") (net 2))
 (segment (start 192.6 132.822159) (end 193.150001 132.272158) (width 0.2) (layer "B.Cu") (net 2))
 (segment (start 203.48 144.09) (end 203.662158 144.272158) (width 0.2) (layer "B.Cu") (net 2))
 (segment (start 212.58 146.64) (end 203.72 146.64) (width 0.2) (layer "B.Cu") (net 2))
 (segment (start 203.662158 144.272158) (end 205.150001 144.272158) (width 0.2) (layer "B.Cu") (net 2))
 (segment (start 235.06 130.65) (end 235.06 133.55) (width 0.2) (layer "B.Cu") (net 2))
 (segment (start 222.56 144.99) (end 222.6 145.03) (width 0.2) (layer "B.Cu") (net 2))
 (segment (start 239 124.5) (end 239.58 124.5) (width 0.2) (layer "F.Cu") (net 4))
 (segment (start 235.665 82.5) (end 239 82.5) (width 0.2) (layer "F.Cu") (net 4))
 (segment (start 239.58 124.5) (end 241.13 126.05) (width 0.2) (layer "F.Cu") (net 4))
 (segment (start 239 82.5) (end 239 124.5) (width 0.2) (layer "F.Cu") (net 4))
 (via (at 241.13 126.05) (size 0.6) (drill 0.3) (layers "F.Cu" "B.Cu") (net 4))
 (segment (start 243.24 132.1) (end 242.0875 132.1) (width 0.2) (layer "B.Cu") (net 4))
 (segment (start 241.13 126.05) (end 243.399 128.319) (width 0.2) (layer "B.Cu") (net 4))
 (segment (start 235.5 80) (end 235.5 81) (width 0.2) (layer "B.Cu") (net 4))
 (segment (start 191.41 127.57) (end 198.35 127.57) (width 0.2) (layer "B.Cu") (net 4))
 (segment (start 235.5 81) (end 235.665 81.165) (width 0.2) (layer "B.Cu") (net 4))
 (segment (start 233.38 148.399) (end 233.38 141.69) (width 0.2) (layer "B.Cu") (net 4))
 (segment (start 203.23 83) (end 203 82.77) (width 0.2) (layer "B.Cu") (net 4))
 (segment (start 211.07 140.73) (end 211.08 140.72) (width 0.2) (layer "B.Cu") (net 4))
 (segment (start 191.101 127.879) (end 191.41 127.57) (width 0.2) (layer "B.Cu") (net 4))
 (segment (start 243.399 128.319) (end 243.399 132.06) (width 0.2) (layer "B.Cu") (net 4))
 (segment (start 243.28 132.06) (end 243.24 132.1) (width 0.2) (layer "B.Cu") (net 4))
 (segment (start 202.77 148.399) (end 202.77 141.16) (width 0.2) (layer "B.Cu") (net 4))
 (segment (start 202.77 148.399) (end 191.101 148.399) (width 0.2) (layer "B.Cu") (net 4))
 (segment (start 243.399 132.06) (end 243.399 147.87) (width 0.2) (layer "B.Cu") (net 4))
 (segment (start 243.399 132.06) (end 243.28 132.06) (width 0.2) (layer "B.Cu") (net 4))
 (segment (start 198.350001 127.569999) (end 198.350001 130.772158) (width 0.2) (layer "B.Cu") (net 4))
 (segment (start 231.7 141.922159) (end 230.850001 142.772158) (width 0.2) (layer "B.Cu") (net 4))
 (segment (start 211.08 140.72) (end 211.08 142.042159) (width 0.2) (layer "B.Cu") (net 4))
 (segment (start 203 80) (end 235.5 80) (width 0.2) (layer "B.Cu") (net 4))
 (segment (start 211.08 142.042159) (end 210.350001 142.772158) (width 0.2) (layer "B.Cu") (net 4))
 (segment (start 233.38 141.69) (end 231.7 140.01) (width 0.2) (layer "B.Cu") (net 4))
 (segment (start 233.38 148.399) (end 202.77 148.399) (width 0.2) (layer "B.Cu") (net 4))
 (segment (start 203 82.27) (end 203 80) (width 0.2) (layer "B.Cu") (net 4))
 (segment (start 243.399 147.87) (end 242.87 148.399) (width 0.2) (layer "B.Cu") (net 4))
 (segment (start 202.77 141.16) (end 203.2 140.73) (width 0.2) (layer "B.Cu") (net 4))
 (segment (start 191.101 148.399) (end 191.101 127.879) (width 0.2) (layer "B.Cu") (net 4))
 (segment (start 235.665 81.165) (end 235.665 82.5) (width 0.2) (layer "B.Cu") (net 4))
 (segment (start 203.2 140.73) (end 211.07 140.73) (width 0.2) (layer "B.Cu") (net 4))
 (segment (start 231.7 140.01) (end 231.7 141.922159) (width 0.2) (layer "B.Cu") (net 4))
 (segment (start 198.35 127.57) (end 198.350001 127.569999) (width 0.2) (layer "B.Cu") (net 4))
 (segment (start 242.87 148.399) (end 233.38 148.399) (width 0.2) (layer "B.Cu") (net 4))
 (segment (start 208.31 83) (end 209.373 81.937) (width 0.2) (layer "B.Cu") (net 13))
 (segment (start 209.5 81.437) (end 220.86531 81.437) (width 0.2) (layer "B.Cu") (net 13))
 (segment (start 209.373 81.937) (end 209.373 81.564) (width 0.2) (layer "B.Cu") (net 13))
 (segment (start 221.901 82.47269) (end 221.901 91.184) (width 0.2) (layer "B.Cu") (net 13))
 (segment (start 209.373 81.564) (end 209.5 81.437) (width 0.2) (layer "B.Cu") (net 13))
 (segment (start 220.86531 81.437) (end 221.901 82.47269) (width 0.2) (layer "B.Cu") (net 13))
 (segment (start 221.901 91.184) (end 220.425 92.66) (width 0.2) (layer "B.Cu") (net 13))
 (segment (start 242.57 147.77) (end 242.28 147.48) (width 0.2) (layer "F.Cu") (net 3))
 (segment (start 242.28 147.48) (end 242.28 135.68) (width 0.2) (layer "F.Cu") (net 3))
 (segment (start 201.48 147.77) (end 242.57 147.77) (width 0.2) (layer "F.Cu") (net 3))
 (segment (start 201.4 147.69) (end 201.48 147.77) (width 0.2) (layer "F.Cu") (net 3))
 (via (at 242.28 135.68) (size 0.6) (drill 0.3) (layers "F.Cu" "B.Cu") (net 3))
 (via (at 201.4 147.69) (size 0.6) (drill 0.3) (layers "F.Cu" "B.Cu") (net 3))
 (segment (start 192.74 128.84) (end 191.94 128.84) (width 0.2) (layer "B.Cu") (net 3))
 (segment (start 242.28 135.68) (end 242.28 135.36) (width 0.2) (layer "B.Cu") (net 3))
 (segment (start 242.0875 135.1675) (end 242.0875 133.6) (width 0.2) (layer "B.Cu") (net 3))
 (segment (start 191.53 147.81) (end 201.28 147.81) (width 0.2) (layer "B.Cu") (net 3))
 (segment (start 242.28 135.36) (end 242.0875 135.1675) (width 0.2) (layer "B.Cu") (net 3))
 (segment (start 191.94 128.84) (end 191.502 129.278) (width 0.2) (layer "B.Cu") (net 3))
 (segment (start 201.28 147.81) (end 201.4 147.69) (width 0.2) (layer "B.Cu") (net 3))
 (segment (start 191.502 129.278) (end 191.502 129.43) (width 0.2) (layer "B.Cu") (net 3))
 (segment (start 193.150001 130.772158) (end 192.74 130.362157) (width 0.2) (layer "B.Cu") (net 3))
 (segment (start 191.502 129.43) (end 191.53 129.458) (width 0.2) (layer "B.Cu") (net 3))
 (segment (start 192.74 130.362157) (end 192.74 128.84) (width 0.2) (layer "B.Cu") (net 3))
 (segment (start 191.53 129.458) (end 191.53 147.81) (width 0.2) (layer "B.Cu") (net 3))
 (segment (start 193.86 90.12) (end 192.5 91.48) (width 0.2) (layer "F.Cu") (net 12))
 (segment (start 220.425 90.12) (end 193.86 90.12) (width 0.2) (layer "F.Cu") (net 12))
 (segment (start 201.842 133.778) (end 197.37 138.25) (width 0.2) (layer "F.Cu") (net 12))
 (segment (start 192.5 91.48) (end 201.842 100.822) (width 0.2) (layer "F.Cu") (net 12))
 (segment (start 201.842 100.822) (end 201.842 133.778) (width 0.2) (layer "F.Cu") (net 12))
 (segment (start 219.59 90.12) (end 220.425 90.12) (width 0.2) (layer "F.Cu") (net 12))
 (via (at 197.37 138.25) (size 0.6) (drill 0.3) (layers "F.Cu" "B.Cu") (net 12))
 (segment (start 198.350001 137.269999) (end 198.350001 132.272158) (width 0.2) (layer "B.Cu") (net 12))
 (segment (start 197.37 138.25) (end 198.350001 137.269999) (width 0.2) (layer "B.Cu") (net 12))
 (segment (start 224.11 137.98) (end 221.38 140.71) (width 0.2) (layer "B.Cu") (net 1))
 (segment (start 234.27 130.590057) (end 234.27 137.98) (width 0.2) (layer "B.Cu") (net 1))
 (segment (start 221.38 140.71) (end 216.28 140.71) (width 0.2) (layer "B.Cu") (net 1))
 (segment (start 212.717842 144.272158) (end 210.350001 144.272158) (width 0.2) (layer "B.Cu") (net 1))
 (segment (start 216.28 140.71) (end 212.717842 144.272158) (width 0.2) (layer "B.Cu") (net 1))
 (segment (start 236.54 128.67) (end 236.190057 128.67) (width 0.2) (layer "B.Cu") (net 1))
 (segment (start 236.8875 132.1) (end 236.8875 129.0175) (width 0.2) (layer "B.Cu") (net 1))
 (segment (start 236.8875 129.0175) (end 236.54 128.67) (width 0.2) (layer "B.Cu") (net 1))
 (segment (start 236.190057 128.67) (end 234.27 130.590057) (width 0.2) (layer "B.Cu") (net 1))
 (segment (start 234.27 137.98) (end 224.11 137.98) (width 0.2) (layer "B.Cu") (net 1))
 (segment (start 214.45 140) (end 221.56 147.11) (width 0.2) (layer "F.Cu") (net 6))
 (segment (start 203.81 141.63) (end 205.44 140) (width 0.2) (layer "F.Cu") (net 6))
 (segment (start 213.8 140) (end 214.45 140) (width 0.2) (layer "F.Cu") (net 6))
 (segment (start 205.44 140) (end 213.8 140) (width 0.2) (layer "F.Cu") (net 6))
 (via (at 203.81 141.63) (size 0.6) (drill 0.3) (layers "F.Cu" "B.Cu") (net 6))
 (via (at 221.56 147.11) (size 0.6) (drill 0.3) (layers "F.Cu" "B.Cu") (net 6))
 (segment (start 205.150001 142.772158) (end 204.952158 142.772158) (width 0.2) (layer "B.Cu") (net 6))
 (segment (start 204.952158 142.772158) (end 203.81 141.63) (width 0.2) (layer "B.Cu") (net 6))
 (segment (start 231.41 144.832157) (end 230.850001 144.272158) (width 0.2) (layer "B.Cu") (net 6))
 (segment (start 231.41 147.06) (end 231.41 144.832157) (width 0.2) (layer "B.Cu") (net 6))
 (segment (start 221.56 147.11) (end 221.61 147.06) (width 0.2) (layer "B.Cu") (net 6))
 (segment (start 221.61 147.06) (end 231.41 147.06) (width 0.2) (layer "B.Cu") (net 6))
 (segment (start 234 114) (end 238 114) (width 0.2) (layer "B.Cu") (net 10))
 (segment (start 218 100.9329) (end 218 89) (width 0.2) (layer "B.Cu") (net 10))
 (segment (start 221.5 89) (end 221.5 86.115) (width 0.2) (layer "B.Cu") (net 10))
 (segment (start 218 89) (end 221.5 89) (width 0.2) (layer "B.Cu") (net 10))
 (segment (start 218.5671 101.5) (end 218 100.9329) (width 0.2) (layer "B.Cu") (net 10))
 (segment (start 238 101.5) (end 218.5671 101.5) (width 0.2) (layer "B.Cu") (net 10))
 (segment (start 238 114) (end 238 101.5) (width 0.2) (layer "B.Cu") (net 10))
 (segment (start 221.5 86.115) (end 220.425 85.04) (width 0.2) (layer "B.Cu") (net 10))
 (segment (start 218.948 87.58) (end 220.425 87.58) (width 0.2) (layer "F.Cu") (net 11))
 (segment (start 217.5 87.5) (end 217.58 87.58) (width 0.2) (layer "B.Cu") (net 11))
 (segment (start 237 102) (end 218.5 102) (width 0.2) (layer "B.Cu") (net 11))
 (segment (start 217.5 101) (end 217.5 87.5) (width 0.2) (layer "B.Cu") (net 11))
 (segment (start 234 109) (end 237 109) (width 0.2) (layer "B.Cu") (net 11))
 (segment (start 218.5 102) (end 217.5 101) (width 0.2) (layer "B.Cu") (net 11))
 (segment (start 217.58 87.58) (end 220.425 87.58) (width 0.2) (layer "B.Cu") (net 11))
 (segment (start 237 109) (end 237 102) (width 0.2) (layer "B.Cu") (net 11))
 (segment (start 219.5 108.5) (end 219.5 98.665) (width 0.2) (layer "F.Cu") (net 15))
 (segment (start 219.5 98.665) (end 220.425 97.74) (width 0.2) (layer "F.Cu") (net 15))
 (segment (start 217 82.5) (end 220.425 82.5) (width 0.2) (layer "B.Cu") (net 9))
 (segment (start 219.5 114) (end 217 114) (width 0.2) (layer "B.Cu") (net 9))
 (segment (start 217 114) (end 217 82.5) (width 0.2) (layer "B.Cu") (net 9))
 (segment (start 239.5 90) (end 239.5 120) (width 0.2) (layer "B.Cu") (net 7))
 (segment (start 235.665 90.12) (end 238.38 90.12) (width 0.2) (layer "B.Cu") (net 7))
 (segment (start 210.663 120.337) (end 210.663 126.954) (width 0.2) (layer "B.Cu") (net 7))
 (segment (start 238.5 90) (end 239.5 90) (width 0.2) (layer "B.Cu") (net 7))
 (segment (start 210.663 120.337) (end 211 120) (width 0.2) (layer "B.Cu") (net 7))
 (segment (start 238.38 90.12) (end 238.5 90) (width 0.2) (layer "B.Cu") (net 7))
 (segment (start 239.5 120) (end 211 120) (width 0.2) (layer "B.Cu") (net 7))
 (segment (start 229.71 98.615) (end 235.665 92.66) (width 0.2) (layer "F.Cu") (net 8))
 (segment (start 229.71 126.92) (end 229.71 98.615) (width 0.2) (layer "F.Cu") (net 8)))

